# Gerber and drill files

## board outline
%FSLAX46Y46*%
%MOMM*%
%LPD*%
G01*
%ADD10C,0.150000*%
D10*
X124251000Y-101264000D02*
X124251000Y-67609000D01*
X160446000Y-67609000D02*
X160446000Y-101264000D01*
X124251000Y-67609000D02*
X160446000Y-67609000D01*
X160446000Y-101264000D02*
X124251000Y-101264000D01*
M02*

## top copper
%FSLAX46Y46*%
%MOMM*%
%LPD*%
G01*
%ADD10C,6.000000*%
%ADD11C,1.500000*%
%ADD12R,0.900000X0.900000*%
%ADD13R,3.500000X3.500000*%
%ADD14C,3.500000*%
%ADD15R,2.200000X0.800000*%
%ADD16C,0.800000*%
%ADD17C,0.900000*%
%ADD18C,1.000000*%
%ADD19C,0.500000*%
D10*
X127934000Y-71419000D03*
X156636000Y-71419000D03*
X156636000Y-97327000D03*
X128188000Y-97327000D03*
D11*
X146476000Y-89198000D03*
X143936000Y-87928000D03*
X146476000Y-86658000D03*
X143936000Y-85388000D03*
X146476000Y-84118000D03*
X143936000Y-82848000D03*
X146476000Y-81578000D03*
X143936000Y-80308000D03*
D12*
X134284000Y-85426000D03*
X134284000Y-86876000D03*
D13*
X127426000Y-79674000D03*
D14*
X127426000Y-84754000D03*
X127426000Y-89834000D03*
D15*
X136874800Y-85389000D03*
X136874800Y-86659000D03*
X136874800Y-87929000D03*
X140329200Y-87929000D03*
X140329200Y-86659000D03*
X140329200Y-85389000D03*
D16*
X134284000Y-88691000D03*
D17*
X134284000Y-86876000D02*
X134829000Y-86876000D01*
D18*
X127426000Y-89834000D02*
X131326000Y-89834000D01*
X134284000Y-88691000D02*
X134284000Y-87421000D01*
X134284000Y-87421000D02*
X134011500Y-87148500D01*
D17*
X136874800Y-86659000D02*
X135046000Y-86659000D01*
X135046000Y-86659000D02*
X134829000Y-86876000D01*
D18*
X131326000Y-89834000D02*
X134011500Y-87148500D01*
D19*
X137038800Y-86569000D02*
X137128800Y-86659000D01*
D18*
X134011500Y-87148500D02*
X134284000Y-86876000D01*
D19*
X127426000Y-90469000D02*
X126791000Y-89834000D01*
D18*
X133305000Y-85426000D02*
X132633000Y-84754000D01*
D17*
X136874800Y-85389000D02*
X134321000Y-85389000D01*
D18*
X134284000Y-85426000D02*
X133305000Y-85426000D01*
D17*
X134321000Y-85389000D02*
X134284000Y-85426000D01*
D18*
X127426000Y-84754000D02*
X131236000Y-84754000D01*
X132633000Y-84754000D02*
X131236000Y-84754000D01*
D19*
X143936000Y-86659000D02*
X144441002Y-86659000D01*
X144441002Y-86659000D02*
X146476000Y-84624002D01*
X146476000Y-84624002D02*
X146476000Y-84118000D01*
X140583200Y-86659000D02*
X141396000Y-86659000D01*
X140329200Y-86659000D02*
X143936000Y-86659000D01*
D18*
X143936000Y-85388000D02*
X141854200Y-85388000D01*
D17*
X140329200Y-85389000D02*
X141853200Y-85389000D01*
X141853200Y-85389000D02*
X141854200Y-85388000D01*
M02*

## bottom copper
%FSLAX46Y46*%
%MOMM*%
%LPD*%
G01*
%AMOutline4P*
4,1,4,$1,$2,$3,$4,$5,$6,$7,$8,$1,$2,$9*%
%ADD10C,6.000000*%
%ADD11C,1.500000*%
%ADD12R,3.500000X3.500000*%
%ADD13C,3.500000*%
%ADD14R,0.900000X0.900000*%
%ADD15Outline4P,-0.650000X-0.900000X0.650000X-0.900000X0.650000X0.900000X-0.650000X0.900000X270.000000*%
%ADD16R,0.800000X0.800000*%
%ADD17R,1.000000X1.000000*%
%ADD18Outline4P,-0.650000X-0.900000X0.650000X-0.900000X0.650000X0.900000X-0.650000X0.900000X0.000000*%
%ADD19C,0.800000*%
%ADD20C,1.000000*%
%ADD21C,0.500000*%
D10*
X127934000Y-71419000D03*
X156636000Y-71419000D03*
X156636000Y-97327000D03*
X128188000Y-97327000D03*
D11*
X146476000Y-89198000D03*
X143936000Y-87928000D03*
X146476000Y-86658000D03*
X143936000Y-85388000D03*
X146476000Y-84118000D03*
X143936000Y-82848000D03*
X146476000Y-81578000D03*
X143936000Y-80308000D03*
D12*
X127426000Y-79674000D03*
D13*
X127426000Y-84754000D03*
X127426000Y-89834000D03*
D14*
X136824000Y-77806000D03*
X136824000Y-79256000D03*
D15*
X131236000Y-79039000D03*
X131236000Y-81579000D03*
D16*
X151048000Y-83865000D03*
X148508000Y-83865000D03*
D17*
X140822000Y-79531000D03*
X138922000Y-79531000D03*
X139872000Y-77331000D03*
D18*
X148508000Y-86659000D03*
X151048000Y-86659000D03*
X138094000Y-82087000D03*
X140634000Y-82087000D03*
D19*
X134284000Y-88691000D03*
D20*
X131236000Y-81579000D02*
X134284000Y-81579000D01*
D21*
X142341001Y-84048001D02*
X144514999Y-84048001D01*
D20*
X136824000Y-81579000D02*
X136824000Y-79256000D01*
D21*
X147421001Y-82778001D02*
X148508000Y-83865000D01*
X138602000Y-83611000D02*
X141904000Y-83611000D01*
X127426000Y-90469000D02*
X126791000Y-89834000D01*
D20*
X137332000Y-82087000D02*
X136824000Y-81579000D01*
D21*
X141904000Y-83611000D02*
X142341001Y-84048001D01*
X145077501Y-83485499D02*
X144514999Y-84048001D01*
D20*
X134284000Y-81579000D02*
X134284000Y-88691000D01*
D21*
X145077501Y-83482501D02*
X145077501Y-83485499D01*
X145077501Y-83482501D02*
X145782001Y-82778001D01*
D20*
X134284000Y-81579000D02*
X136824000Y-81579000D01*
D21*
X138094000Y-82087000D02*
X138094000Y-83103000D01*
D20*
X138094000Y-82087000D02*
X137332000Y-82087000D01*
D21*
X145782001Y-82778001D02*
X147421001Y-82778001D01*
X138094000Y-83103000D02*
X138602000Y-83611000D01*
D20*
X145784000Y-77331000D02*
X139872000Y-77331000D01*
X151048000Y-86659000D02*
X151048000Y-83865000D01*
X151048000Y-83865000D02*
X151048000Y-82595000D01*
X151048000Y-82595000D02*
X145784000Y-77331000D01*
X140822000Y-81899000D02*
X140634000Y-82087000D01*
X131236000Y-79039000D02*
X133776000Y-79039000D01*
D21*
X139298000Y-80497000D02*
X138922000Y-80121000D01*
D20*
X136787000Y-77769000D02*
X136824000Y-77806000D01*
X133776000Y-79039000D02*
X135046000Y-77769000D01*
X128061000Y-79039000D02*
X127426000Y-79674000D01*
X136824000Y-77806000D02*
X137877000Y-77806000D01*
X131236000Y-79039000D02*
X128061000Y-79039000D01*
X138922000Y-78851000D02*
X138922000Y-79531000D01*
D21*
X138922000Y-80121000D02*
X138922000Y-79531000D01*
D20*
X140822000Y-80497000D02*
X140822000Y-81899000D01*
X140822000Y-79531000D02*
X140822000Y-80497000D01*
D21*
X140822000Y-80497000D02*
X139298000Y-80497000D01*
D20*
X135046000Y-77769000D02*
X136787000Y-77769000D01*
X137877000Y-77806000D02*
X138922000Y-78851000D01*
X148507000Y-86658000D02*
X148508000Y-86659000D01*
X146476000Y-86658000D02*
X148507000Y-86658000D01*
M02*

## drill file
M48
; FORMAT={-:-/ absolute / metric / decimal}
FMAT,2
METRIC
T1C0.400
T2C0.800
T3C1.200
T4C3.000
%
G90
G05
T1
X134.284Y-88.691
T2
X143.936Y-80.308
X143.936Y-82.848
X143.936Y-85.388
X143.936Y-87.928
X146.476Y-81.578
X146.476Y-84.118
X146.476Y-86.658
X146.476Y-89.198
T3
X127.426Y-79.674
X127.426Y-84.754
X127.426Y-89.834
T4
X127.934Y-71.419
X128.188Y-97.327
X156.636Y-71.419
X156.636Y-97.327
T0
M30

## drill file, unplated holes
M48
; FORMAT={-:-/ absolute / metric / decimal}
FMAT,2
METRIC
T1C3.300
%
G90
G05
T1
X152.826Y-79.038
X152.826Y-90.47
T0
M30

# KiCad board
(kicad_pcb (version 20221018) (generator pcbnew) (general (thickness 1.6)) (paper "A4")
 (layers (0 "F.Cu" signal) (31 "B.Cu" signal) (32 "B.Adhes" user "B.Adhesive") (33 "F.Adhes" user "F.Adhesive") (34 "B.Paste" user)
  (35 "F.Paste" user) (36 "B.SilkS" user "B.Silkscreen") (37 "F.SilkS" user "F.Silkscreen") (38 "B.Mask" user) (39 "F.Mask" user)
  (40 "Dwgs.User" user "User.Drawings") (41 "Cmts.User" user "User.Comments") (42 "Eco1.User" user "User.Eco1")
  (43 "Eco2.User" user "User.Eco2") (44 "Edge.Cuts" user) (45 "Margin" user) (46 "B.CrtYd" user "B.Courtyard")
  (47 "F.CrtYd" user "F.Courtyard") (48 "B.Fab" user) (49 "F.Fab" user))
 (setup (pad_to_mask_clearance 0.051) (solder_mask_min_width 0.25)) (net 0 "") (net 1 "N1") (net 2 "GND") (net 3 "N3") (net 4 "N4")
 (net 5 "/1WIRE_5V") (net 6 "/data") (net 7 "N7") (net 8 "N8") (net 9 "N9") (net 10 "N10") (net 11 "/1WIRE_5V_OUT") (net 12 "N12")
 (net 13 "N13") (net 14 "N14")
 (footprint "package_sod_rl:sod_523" (layer "F.Cu") (at 134.284 86.151 -90)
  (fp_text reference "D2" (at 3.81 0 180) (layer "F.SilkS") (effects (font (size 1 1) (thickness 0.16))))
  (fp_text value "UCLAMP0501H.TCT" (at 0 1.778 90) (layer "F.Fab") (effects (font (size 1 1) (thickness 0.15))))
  (pad "1" smd rect (at -0.725 0 270) (size 0.9 0.9) (layers "F.Cu" "F.Paste" "F.Mask") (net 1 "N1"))
  (pad "2" smd rect (at 0.725 0 270) (size 0.9 0.9) (layers "F.Cu" "F.Paste" "F.Mask") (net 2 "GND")))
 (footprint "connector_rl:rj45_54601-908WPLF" (layer "F.Cu") (at 152.826 84.754 90)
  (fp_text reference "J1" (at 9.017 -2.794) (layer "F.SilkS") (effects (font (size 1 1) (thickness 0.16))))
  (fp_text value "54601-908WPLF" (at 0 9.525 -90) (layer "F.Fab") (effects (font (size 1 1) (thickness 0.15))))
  (pad "" np_thru_hole circle (at -5.716 0 90) (size 3.3 3.3) (drill 3.3) (layers "*.Cu" "*.SilkS" "*.Mask"))
  (pad "" np_thru_hole circle (at 5.716 0 90) (size 3.3 3.3) (drill 3.3) (layers "*.Cu" "*.SilkS" "*.Mask"))
  (pad "1" thru_hole circle (at -4.444 -6.35 90) (size 1.5 1.5) (drill 0.8) (layers "*.Cu" "*.Mask") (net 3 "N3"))
  (pad "2" thru_hole circle (at -3.174 -8.89 90) (size 1.5 1.5) (drill 0.8) (layers "*.Cu" "*.Mask") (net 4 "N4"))
  (pad "3" thru_hole circle (at -1.904 -6.35 90) (size 1.5 1.5) (drill 0.8) (layers "*.Cu" "*.Mask") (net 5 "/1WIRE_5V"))
  (pad "4" thru_hole circle (at -0.634 -8.89 90) (size 1.5 1.5) (drill 0.8) (layers "*.Cu" "*.Mask") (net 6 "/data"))
  (pad "5" thru_hole circle (at 0.636 -6.35 90) (size 1.5 1.5) (drill 0.8) (layers "*.Cu" "*.Mask") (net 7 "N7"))
  (pad "6" thru_hole circle (at 1.906 -8.89 270) (size 1.5 1.5) (drill 0.8) (layers "*.Cu" "*.Mask") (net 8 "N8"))
  (pad "7" thru_hole circle (at 3.176 -6.35 90) (size 1.5 1.5) (drill 0.8) (layers "*.Cu" "*.Mask") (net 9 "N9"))
  (pad "8" thru_hole circle (at 4.446 -8.89 90) (size 1.5 1.5) (drill 0.8) (layers "*.Cu" "*.Mask") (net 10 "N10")))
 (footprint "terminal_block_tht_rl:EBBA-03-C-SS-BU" (layer "F.Cu") (at 127.426 84.754 -90)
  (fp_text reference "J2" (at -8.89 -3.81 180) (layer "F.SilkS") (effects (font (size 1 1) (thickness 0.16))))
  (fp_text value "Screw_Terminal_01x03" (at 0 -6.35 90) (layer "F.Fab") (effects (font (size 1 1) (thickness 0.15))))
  (pad "1" thru_hole rect (at -5.08 0 90) (size 3.5 3.5) (drill 1.2) (layers "*.Cu" "*.Mask") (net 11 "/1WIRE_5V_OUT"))
  (pad "2" thru_hole circle (at 0 0 90) (size 3.5 3.5) (drill 1.2) (layers "*.Cu" "*.Mask") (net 1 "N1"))
  (pad "3" thru_hole circle (at 5.08 0 90) (size 3.5 3.5) (drill 1.2) (layers "*.Cu" "*.Mask") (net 2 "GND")))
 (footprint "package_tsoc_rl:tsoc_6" (layer "F.Cu") (at 138.602 86.659)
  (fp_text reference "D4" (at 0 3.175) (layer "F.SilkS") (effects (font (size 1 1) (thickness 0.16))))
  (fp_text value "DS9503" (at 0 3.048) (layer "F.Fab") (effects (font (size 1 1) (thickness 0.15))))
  (pad "1" smd rect (at -1.7272 -1.27) (size 2.2 0.8) (layers "F.Cu" "F.Paste" "F.Mask") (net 1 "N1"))
  (pad "2" smd rect (at -1.7272 0) (size 2.2 0.8) (layers "F.Cu" "F.Paste" "F.Mask") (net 2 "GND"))
  (pad "3" smd rect (at -1.7272 1.27) (size 2.2 0.8) (layers "F.Cu" "F.Paste" "F.Mask") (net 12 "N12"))
  (pad "4" smd rect (at 1.7272 1.27) (size 2.2 0.8) (layers "F.Cu" "F.Paste" "F.Mask") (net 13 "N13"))
  (pad "5" smd rect (at 1.7272 0) (size 2.2 0.8) (layers "F.Cu" "F.Paste" "F.Mask") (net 7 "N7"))
  (pad "6" smd rect (at 1.7272 -1.27) (size 2.2 0.8) (layers "F.Cu" "F.Paste" "F.Mask") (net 6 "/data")))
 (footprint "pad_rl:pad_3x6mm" (layer "F.Cu") (at 127.934 71.419)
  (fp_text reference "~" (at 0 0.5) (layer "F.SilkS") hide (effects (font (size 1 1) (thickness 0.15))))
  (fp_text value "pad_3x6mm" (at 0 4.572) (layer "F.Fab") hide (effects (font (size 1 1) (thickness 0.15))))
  (pad "~" thru_hole circle (at 0 0) (size 6 6) (drill 3) (layers "*.Cu" "*.Mask")))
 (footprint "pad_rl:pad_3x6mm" (layer "F.Cu") (at 156.636 71.419)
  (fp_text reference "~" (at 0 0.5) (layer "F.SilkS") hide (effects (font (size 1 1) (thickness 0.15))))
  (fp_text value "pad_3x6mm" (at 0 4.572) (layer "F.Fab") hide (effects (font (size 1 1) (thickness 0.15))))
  (pad "~" thru_hole circle (at 0 0) (size 6 6) (drill 3) (layers "*.Cu" "*.Mask")))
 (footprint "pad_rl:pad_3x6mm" (layer "F.Cu") (at 156.636 97.327)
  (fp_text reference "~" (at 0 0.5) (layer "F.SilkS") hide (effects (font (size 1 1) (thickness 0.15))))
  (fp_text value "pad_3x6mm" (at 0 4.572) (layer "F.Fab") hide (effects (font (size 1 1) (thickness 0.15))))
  (pad "~" thru_hole circle (at 0 0) (size 6 6) (drill 3) (layers "*.Cu" "*.Mask")))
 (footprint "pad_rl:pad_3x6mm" (layer "F.Cu") (at 128.188 97.327)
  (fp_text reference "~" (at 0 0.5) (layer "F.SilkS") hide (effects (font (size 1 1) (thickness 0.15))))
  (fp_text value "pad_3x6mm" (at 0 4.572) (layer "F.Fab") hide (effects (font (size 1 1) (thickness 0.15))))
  (pad "~" thru_hole circle (at 0 0) (size 6 6) (drill 3) (layers "*.Cu" "*.Mask")))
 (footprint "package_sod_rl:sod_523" (layer "B.Cu") (at 136.824 78.531 -90)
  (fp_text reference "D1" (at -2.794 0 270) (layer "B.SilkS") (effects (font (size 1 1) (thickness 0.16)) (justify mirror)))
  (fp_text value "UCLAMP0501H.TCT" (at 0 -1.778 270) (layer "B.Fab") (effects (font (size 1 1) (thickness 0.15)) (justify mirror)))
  (pad "1" smd rect (at -0.725 0 270) (size 0.9 0.9) (layers "B.Cu" "B.Paste" "B.Mask") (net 11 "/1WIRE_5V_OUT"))
  (pad "2" smd rect (at 0.725 0 270) (size 0.9 0.9) (layers "B.Cu" "B.Paste" "B.Mask") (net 2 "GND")))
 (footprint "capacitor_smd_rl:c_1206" (layer "B.Cu") (at 131.236 80.309 -90)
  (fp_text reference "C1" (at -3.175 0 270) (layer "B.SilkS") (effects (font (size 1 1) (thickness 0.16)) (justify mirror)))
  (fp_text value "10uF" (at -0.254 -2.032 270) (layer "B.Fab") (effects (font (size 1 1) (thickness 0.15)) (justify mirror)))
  (pad "1" smd trapezoid (at -1.27 0 270) (size 1.3 1.8) (layers "B.Cu" "B.Paste" "B.Mask") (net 11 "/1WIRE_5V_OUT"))
  (pad "2" smd trapezoid (at 1.27 0 270) (size 1.3 1.8) (layers "B.Cu" "B.Paste" "B.Mask") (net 2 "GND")))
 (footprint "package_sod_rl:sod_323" (layer "B.Cu") (at 149.778 83.865 180)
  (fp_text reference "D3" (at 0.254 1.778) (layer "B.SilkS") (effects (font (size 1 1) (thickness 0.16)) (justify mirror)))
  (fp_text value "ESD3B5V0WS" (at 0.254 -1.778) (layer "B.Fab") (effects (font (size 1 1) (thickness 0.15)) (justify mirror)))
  (pad "1" smd rect (at -1.27 0 180) (size 0.8 0.8) (layers "B.Cu" "B.Paste" "B.Mask") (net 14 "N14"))
  (pad "2" smd rect (at 1.27 0 180) (size 0.8 0.8) (layers "B.Cu" "B.Paste" "B.Mask") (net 2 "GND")))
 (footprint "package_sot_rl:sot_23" (layer "B.Cu") (at 139.872 78.531 90)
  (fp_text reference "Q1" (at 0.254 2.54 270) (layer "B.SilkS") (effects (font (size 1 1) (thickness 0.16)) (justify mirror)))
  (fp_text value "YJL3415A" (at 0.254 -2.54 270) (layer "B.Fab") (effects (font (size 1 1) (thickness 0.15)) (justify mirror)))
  (pad "1" smd rect (at -1 0.95 90) (size 1 1) (layers "B.Cu" "B.Paste" "B.Mask") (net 11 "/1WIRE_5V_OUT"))
  (pad "2" smd rect (at -1 -0.95 90) (size 1 1) (layers "B.Cu" "B.Paste" "B.Mask") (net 11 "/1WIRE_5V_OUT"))
  (pad "3" smd rect (at 1.2 0 90) (size 1 1) (layers "B.Cu" "B.Paste" "B.Mask") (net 14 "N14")))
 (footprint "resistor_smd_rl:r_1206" (layer "B.Cu") (at 149.778 86.659)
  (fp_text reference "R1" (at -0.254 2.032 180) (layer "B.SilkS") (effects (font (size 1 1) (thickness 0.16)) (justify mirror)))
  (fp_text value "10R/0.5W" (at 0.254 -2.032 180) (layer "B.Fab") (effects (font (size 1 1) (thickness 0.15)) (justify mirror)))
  (pad "1" smd trapezoid (at -1.27 0) (size 1.3 1.8) (layers "B.Cu" "B.Paste" "B.Mask") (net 5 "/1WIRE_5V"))
  (pad "2" smd trapezoid (at 1.27 0) (size 1.3 1.8) (layers "B.Cu" "B.Paste" "B.Mask") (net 14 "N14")))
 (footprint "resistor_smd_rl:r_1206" (layer "B.Cu") (at 139.364 82.087)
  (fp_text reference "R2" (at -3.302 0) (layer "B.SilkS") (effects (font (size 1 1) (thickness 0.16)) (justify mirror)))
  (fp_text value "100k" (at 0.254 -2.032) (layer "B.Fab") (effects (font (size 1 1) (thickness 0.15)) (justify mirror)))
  (pad "1" smd trapezoid (at -1.27 0) (size 1.3 1.8) (layers "B.Cu" "B.Paste" "B.Mask") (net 2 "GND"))
  (pad "2" smd trapezoid (at 1.27 0) (size 1.3 1.8) (layers "B.Cu" "B.Paste" "B.Mask") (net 11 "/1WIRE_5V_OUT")))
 (gr_line (start 124.251 101.264) (end 124.251 67.609) (stroke (width 0.15) (type solid)) (layer "Edge.Cuts"))
 (gr_line (start 160.446 67.609) (end 160.446 101.264) (stroke (width 0.15) (type solid)) (layer "Edge.Cuts"))
 (gr_line (start 124.251 67.609) (end 160.446 67.609) (stroke (width 0.15) (type solid)) (layer "Edge.Cuts"))
 (gr_line (start 160.446 101.264) (end 124.251 101.264) (stroke (width 0.15) (type solid)) (layer "Edge.Cuts"))
 (segment (start 134.284 86.876) (end 134.829 86.876) (width 0.9) (layer "F.Cu") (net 2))
 (segment (start 127.426 89.834) (end 131.326 89.834) (width 1) (layer "F.Cu") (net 2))
 (segment (start 134.284 88.691) (end 134.284 87.421) (width 1) (layer "F.Cu") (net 2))
 (segment (start 134.284 87.421) (end 134.0115 87.1485) (width 1) (layer "F.Cu") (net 2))
 (segment (start 136.8748 86.659) (end 135.046 86.659) (width 0.9) (layer "F.Cu") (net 2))
 (segment (start 135.046 86.659) (end 134.829 86.876) (width 0.9) (layer "F.Cu") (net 2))
 (segment (start 131.326 89.834) (end 134.0115 87.1485) (width 1) (layer "F.Cu") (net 2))
 (segment (start 137.0388 86.569) (end 137.1288 86.659) (width 0.5) (layer "F.Cu") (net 2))
 (segment (start 134.0115 87.1485) (end 134.284 86.876) (width 1) (layer "F.Cu") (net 2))
 (segment (start 127.426 90.469) (end 126.791 89.834) (width 0.5) (layer "F.Cu") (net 2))
 (via (at 134.284 88.691) (size 0.8) (drill 0.4) (layers "F.Cu" "B.Cu") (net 2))
 (segment (start 131.236 81.579) (end 134.284 81.579) (width 1) (layer "B.Cu") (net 2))
 (segment (start 142.341001 84.048001) (end 144.514999 84.048001) (width 0.5) (layer "B.Cu") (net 2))
 (segment (start 136.824 81.579) (end 136.824 79.256) (width 1) (layer "B.Cu") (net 2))
 (segment (start 147.421001 82.778001) (end 148.508 83.865) (width 0.5) (layer "B.Cu") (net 2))
 (segment (start 138.602 83.611) (end 141.904 83.611) (width 0.5) (layer "B.Cu") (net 2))
 (segment (start 127.426 90.469) (end 126.791 89.834) (width 0.5) (layer "B.Cu") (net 2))
 (segment (start 137.332 82.087) (end 136.824 81.579) (width 1) (layer "B.Cu") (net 2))
 (segment (start 141.904 83.611) (end 142.341001 84.048001) (width 0.5) (layer "B.Cu") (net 2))
 (segment (start 145.077501 83.485499) (end 144.514999 84.048001) (width 0.5) (layer "B.Cu") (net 2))
 (segment (start 134.284 81.579) (end 134.284 88.691) (width 1) (layer "B.Cu") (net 2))
 (segment (start 145.077501 83.482501) (end 145.077501 83.485499) (width 0.5) (layer "B.Cu") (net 2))
 (segment (start 145.077501 83.482501) (end 145.782001 82.778001) (width 0.5) (layer "B.Cu") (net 2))
 (segment (start 134.284 81.579) (end 136.824 81.579) (width 1) (layer "B.Cu") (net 2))
 (segment (start 138.094 82.087) (end 138.094 83.103) (width 0.5) (layer "B.Cu") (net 2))
 (segment (start 138.094 82.087) (end 137.332 82.087) (width 1) (layer "B.Cu") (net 2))
 (segment (start 145.782001 82.778001) (end 147.421001 82.778001) (width 0.5) (layer "B.Cu") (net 2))
 (segment (start 138.094 83.103) (end 138.602 83.611) (width 0.5) (layer "B.Cu") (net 2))
 (segment (start 133.305 85.426) (end 132.633 84.754) (width 1) (layer "F.Cu") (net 1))
 (segment (start 136.8748 85.389) (end 134.321 85.389) (width 0.9) (layer "F.Cu") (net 1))
 (segment (start 134.284 85.426) (end 133.305 85.426) (width 1) (layer "F.Cu") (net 1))
 (segment (start 134.321 85.389) (end 134.284 85.426) (width 0.9) (layer "F.Cu") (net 1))
 (segment (start 127.426 84.754) (end 131.236 84.754) (width 1) (layer "F.Cu") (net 1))
 (segment (start 132.633 84.754) (end 131.236 84.754) (width 1) (layer "F.Cu") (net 1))
 (segment (start 145.784 77.331) (end 139.872 77.331) (width 1) (layer "B.Cu") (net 14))
 (segment (start 151.048 86.659) (end 151.048 83.865) (width 1) (layer "B.Cu") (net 14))
 (segment (start 151.048 83.865) (end 151.048 82.595) (width 1) (layer "B.Cu") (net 14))
 (segment (start 151.048 82.595) (end 145.784 77.331) (width 1) (layer "B.Cu") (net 14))
 (segment (start 143.936 86.659) (end 144.441002 86.659) (width 0.5) (layer "F.Cu") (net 7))
 (segment (start 144.441002 86.659) (end 146.476 84.624002) (width 0.5) (layer "F.Cu") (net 7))
 (segment (start 146.476 84.624002) (end 146.476 84.118) (width 0.5) (layer "F.Cu") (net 7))
 (segment (start 140.5832 86.659) (end 141.396 86.659) (width 0.5) (layer "F.Cu") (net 7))
 (segment (start 140.3292 86.659) (end 143.936 86.659) (width 0.5) (layer "F.Cu") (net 7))
 (segment (start 143.936 85.388) (end 141.8542 85.388) (width 1) (layer "F.Cu") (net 6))
 (segment (start 140.3292 85.389) (end 141.8532 85.389) (width 0.9) (layer "F.Cu") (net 6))
 (segment (start 141.8532 85.389) (end 141.8542 85.388) (width 0.9) (layer "F.Cu") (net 6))
 (segment (start 140.822 81.899) (end 140.634 82.087) (width 1) (layer "B.Cu") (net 11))
 (segment (start 131.236 79.039) (end 133.776 79.039) (width 1) (layer "B.Cu") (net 11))
 (segment (start 139.298 80.497) (end 138.922 80.121) (width 0.5) (layer "B.Cu") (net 11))
 (segment (start 136.787 77.769) (end 136.824 77.806) (width 1) (layer "B.Cu") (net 11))
 (segment (start 133.776 79.039) (end 135.046 77.769) (width 1) (layer "B.Cu") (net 11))
 (segment (start 128.061 79.039) (end 127.426 79.674) (width 1) (layer "B.Cu") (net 11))
 (segment (start 136.824 77.806) (end 137.877 77.806) (width 1) (layer "B.Cu") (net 11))
 (segment (start 131.236 79.039) (end 128.061 79.039) (width 1) (layer "B.Cu") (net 11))
 (segment (start 138.922 78.851) (end 138.922 79.531) (width 1) (layer "B.Cu") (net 11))
 (segment (start 138.922 80.121) (end 138.922 79.531) (width 0.5) (layer "B.Cu") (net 11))
 (segment (start 140.822 80.497) (end 140.822 81.899) (width 1) (layer "B.Cu") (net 11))
 (segment (start 140.822 79.531) (end 140.822 80.497) (width 1) (layer "B.Cu") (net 11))
 (segment (start 140.822 80.497) (end 139.298 80.497) (width 0.5) (layer "B.Cu") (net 11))
 (segment (start 135.046 77.769) (end 136.787 77.769) (width 1) (layer "B.Cu") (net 11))
 (segment (start 137.877 77.806) (end 138.922 78.851) (width 1) (layer "B.Cu") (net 11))
 (segment (start 148.507 86.658) (end 148.508 86.659) (width 1) (layer "B.Cu") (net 5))
 (segment (start 146.476 86.658) (end 148.507 86.658) (width 1) (layer "B.Cu") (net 5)))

